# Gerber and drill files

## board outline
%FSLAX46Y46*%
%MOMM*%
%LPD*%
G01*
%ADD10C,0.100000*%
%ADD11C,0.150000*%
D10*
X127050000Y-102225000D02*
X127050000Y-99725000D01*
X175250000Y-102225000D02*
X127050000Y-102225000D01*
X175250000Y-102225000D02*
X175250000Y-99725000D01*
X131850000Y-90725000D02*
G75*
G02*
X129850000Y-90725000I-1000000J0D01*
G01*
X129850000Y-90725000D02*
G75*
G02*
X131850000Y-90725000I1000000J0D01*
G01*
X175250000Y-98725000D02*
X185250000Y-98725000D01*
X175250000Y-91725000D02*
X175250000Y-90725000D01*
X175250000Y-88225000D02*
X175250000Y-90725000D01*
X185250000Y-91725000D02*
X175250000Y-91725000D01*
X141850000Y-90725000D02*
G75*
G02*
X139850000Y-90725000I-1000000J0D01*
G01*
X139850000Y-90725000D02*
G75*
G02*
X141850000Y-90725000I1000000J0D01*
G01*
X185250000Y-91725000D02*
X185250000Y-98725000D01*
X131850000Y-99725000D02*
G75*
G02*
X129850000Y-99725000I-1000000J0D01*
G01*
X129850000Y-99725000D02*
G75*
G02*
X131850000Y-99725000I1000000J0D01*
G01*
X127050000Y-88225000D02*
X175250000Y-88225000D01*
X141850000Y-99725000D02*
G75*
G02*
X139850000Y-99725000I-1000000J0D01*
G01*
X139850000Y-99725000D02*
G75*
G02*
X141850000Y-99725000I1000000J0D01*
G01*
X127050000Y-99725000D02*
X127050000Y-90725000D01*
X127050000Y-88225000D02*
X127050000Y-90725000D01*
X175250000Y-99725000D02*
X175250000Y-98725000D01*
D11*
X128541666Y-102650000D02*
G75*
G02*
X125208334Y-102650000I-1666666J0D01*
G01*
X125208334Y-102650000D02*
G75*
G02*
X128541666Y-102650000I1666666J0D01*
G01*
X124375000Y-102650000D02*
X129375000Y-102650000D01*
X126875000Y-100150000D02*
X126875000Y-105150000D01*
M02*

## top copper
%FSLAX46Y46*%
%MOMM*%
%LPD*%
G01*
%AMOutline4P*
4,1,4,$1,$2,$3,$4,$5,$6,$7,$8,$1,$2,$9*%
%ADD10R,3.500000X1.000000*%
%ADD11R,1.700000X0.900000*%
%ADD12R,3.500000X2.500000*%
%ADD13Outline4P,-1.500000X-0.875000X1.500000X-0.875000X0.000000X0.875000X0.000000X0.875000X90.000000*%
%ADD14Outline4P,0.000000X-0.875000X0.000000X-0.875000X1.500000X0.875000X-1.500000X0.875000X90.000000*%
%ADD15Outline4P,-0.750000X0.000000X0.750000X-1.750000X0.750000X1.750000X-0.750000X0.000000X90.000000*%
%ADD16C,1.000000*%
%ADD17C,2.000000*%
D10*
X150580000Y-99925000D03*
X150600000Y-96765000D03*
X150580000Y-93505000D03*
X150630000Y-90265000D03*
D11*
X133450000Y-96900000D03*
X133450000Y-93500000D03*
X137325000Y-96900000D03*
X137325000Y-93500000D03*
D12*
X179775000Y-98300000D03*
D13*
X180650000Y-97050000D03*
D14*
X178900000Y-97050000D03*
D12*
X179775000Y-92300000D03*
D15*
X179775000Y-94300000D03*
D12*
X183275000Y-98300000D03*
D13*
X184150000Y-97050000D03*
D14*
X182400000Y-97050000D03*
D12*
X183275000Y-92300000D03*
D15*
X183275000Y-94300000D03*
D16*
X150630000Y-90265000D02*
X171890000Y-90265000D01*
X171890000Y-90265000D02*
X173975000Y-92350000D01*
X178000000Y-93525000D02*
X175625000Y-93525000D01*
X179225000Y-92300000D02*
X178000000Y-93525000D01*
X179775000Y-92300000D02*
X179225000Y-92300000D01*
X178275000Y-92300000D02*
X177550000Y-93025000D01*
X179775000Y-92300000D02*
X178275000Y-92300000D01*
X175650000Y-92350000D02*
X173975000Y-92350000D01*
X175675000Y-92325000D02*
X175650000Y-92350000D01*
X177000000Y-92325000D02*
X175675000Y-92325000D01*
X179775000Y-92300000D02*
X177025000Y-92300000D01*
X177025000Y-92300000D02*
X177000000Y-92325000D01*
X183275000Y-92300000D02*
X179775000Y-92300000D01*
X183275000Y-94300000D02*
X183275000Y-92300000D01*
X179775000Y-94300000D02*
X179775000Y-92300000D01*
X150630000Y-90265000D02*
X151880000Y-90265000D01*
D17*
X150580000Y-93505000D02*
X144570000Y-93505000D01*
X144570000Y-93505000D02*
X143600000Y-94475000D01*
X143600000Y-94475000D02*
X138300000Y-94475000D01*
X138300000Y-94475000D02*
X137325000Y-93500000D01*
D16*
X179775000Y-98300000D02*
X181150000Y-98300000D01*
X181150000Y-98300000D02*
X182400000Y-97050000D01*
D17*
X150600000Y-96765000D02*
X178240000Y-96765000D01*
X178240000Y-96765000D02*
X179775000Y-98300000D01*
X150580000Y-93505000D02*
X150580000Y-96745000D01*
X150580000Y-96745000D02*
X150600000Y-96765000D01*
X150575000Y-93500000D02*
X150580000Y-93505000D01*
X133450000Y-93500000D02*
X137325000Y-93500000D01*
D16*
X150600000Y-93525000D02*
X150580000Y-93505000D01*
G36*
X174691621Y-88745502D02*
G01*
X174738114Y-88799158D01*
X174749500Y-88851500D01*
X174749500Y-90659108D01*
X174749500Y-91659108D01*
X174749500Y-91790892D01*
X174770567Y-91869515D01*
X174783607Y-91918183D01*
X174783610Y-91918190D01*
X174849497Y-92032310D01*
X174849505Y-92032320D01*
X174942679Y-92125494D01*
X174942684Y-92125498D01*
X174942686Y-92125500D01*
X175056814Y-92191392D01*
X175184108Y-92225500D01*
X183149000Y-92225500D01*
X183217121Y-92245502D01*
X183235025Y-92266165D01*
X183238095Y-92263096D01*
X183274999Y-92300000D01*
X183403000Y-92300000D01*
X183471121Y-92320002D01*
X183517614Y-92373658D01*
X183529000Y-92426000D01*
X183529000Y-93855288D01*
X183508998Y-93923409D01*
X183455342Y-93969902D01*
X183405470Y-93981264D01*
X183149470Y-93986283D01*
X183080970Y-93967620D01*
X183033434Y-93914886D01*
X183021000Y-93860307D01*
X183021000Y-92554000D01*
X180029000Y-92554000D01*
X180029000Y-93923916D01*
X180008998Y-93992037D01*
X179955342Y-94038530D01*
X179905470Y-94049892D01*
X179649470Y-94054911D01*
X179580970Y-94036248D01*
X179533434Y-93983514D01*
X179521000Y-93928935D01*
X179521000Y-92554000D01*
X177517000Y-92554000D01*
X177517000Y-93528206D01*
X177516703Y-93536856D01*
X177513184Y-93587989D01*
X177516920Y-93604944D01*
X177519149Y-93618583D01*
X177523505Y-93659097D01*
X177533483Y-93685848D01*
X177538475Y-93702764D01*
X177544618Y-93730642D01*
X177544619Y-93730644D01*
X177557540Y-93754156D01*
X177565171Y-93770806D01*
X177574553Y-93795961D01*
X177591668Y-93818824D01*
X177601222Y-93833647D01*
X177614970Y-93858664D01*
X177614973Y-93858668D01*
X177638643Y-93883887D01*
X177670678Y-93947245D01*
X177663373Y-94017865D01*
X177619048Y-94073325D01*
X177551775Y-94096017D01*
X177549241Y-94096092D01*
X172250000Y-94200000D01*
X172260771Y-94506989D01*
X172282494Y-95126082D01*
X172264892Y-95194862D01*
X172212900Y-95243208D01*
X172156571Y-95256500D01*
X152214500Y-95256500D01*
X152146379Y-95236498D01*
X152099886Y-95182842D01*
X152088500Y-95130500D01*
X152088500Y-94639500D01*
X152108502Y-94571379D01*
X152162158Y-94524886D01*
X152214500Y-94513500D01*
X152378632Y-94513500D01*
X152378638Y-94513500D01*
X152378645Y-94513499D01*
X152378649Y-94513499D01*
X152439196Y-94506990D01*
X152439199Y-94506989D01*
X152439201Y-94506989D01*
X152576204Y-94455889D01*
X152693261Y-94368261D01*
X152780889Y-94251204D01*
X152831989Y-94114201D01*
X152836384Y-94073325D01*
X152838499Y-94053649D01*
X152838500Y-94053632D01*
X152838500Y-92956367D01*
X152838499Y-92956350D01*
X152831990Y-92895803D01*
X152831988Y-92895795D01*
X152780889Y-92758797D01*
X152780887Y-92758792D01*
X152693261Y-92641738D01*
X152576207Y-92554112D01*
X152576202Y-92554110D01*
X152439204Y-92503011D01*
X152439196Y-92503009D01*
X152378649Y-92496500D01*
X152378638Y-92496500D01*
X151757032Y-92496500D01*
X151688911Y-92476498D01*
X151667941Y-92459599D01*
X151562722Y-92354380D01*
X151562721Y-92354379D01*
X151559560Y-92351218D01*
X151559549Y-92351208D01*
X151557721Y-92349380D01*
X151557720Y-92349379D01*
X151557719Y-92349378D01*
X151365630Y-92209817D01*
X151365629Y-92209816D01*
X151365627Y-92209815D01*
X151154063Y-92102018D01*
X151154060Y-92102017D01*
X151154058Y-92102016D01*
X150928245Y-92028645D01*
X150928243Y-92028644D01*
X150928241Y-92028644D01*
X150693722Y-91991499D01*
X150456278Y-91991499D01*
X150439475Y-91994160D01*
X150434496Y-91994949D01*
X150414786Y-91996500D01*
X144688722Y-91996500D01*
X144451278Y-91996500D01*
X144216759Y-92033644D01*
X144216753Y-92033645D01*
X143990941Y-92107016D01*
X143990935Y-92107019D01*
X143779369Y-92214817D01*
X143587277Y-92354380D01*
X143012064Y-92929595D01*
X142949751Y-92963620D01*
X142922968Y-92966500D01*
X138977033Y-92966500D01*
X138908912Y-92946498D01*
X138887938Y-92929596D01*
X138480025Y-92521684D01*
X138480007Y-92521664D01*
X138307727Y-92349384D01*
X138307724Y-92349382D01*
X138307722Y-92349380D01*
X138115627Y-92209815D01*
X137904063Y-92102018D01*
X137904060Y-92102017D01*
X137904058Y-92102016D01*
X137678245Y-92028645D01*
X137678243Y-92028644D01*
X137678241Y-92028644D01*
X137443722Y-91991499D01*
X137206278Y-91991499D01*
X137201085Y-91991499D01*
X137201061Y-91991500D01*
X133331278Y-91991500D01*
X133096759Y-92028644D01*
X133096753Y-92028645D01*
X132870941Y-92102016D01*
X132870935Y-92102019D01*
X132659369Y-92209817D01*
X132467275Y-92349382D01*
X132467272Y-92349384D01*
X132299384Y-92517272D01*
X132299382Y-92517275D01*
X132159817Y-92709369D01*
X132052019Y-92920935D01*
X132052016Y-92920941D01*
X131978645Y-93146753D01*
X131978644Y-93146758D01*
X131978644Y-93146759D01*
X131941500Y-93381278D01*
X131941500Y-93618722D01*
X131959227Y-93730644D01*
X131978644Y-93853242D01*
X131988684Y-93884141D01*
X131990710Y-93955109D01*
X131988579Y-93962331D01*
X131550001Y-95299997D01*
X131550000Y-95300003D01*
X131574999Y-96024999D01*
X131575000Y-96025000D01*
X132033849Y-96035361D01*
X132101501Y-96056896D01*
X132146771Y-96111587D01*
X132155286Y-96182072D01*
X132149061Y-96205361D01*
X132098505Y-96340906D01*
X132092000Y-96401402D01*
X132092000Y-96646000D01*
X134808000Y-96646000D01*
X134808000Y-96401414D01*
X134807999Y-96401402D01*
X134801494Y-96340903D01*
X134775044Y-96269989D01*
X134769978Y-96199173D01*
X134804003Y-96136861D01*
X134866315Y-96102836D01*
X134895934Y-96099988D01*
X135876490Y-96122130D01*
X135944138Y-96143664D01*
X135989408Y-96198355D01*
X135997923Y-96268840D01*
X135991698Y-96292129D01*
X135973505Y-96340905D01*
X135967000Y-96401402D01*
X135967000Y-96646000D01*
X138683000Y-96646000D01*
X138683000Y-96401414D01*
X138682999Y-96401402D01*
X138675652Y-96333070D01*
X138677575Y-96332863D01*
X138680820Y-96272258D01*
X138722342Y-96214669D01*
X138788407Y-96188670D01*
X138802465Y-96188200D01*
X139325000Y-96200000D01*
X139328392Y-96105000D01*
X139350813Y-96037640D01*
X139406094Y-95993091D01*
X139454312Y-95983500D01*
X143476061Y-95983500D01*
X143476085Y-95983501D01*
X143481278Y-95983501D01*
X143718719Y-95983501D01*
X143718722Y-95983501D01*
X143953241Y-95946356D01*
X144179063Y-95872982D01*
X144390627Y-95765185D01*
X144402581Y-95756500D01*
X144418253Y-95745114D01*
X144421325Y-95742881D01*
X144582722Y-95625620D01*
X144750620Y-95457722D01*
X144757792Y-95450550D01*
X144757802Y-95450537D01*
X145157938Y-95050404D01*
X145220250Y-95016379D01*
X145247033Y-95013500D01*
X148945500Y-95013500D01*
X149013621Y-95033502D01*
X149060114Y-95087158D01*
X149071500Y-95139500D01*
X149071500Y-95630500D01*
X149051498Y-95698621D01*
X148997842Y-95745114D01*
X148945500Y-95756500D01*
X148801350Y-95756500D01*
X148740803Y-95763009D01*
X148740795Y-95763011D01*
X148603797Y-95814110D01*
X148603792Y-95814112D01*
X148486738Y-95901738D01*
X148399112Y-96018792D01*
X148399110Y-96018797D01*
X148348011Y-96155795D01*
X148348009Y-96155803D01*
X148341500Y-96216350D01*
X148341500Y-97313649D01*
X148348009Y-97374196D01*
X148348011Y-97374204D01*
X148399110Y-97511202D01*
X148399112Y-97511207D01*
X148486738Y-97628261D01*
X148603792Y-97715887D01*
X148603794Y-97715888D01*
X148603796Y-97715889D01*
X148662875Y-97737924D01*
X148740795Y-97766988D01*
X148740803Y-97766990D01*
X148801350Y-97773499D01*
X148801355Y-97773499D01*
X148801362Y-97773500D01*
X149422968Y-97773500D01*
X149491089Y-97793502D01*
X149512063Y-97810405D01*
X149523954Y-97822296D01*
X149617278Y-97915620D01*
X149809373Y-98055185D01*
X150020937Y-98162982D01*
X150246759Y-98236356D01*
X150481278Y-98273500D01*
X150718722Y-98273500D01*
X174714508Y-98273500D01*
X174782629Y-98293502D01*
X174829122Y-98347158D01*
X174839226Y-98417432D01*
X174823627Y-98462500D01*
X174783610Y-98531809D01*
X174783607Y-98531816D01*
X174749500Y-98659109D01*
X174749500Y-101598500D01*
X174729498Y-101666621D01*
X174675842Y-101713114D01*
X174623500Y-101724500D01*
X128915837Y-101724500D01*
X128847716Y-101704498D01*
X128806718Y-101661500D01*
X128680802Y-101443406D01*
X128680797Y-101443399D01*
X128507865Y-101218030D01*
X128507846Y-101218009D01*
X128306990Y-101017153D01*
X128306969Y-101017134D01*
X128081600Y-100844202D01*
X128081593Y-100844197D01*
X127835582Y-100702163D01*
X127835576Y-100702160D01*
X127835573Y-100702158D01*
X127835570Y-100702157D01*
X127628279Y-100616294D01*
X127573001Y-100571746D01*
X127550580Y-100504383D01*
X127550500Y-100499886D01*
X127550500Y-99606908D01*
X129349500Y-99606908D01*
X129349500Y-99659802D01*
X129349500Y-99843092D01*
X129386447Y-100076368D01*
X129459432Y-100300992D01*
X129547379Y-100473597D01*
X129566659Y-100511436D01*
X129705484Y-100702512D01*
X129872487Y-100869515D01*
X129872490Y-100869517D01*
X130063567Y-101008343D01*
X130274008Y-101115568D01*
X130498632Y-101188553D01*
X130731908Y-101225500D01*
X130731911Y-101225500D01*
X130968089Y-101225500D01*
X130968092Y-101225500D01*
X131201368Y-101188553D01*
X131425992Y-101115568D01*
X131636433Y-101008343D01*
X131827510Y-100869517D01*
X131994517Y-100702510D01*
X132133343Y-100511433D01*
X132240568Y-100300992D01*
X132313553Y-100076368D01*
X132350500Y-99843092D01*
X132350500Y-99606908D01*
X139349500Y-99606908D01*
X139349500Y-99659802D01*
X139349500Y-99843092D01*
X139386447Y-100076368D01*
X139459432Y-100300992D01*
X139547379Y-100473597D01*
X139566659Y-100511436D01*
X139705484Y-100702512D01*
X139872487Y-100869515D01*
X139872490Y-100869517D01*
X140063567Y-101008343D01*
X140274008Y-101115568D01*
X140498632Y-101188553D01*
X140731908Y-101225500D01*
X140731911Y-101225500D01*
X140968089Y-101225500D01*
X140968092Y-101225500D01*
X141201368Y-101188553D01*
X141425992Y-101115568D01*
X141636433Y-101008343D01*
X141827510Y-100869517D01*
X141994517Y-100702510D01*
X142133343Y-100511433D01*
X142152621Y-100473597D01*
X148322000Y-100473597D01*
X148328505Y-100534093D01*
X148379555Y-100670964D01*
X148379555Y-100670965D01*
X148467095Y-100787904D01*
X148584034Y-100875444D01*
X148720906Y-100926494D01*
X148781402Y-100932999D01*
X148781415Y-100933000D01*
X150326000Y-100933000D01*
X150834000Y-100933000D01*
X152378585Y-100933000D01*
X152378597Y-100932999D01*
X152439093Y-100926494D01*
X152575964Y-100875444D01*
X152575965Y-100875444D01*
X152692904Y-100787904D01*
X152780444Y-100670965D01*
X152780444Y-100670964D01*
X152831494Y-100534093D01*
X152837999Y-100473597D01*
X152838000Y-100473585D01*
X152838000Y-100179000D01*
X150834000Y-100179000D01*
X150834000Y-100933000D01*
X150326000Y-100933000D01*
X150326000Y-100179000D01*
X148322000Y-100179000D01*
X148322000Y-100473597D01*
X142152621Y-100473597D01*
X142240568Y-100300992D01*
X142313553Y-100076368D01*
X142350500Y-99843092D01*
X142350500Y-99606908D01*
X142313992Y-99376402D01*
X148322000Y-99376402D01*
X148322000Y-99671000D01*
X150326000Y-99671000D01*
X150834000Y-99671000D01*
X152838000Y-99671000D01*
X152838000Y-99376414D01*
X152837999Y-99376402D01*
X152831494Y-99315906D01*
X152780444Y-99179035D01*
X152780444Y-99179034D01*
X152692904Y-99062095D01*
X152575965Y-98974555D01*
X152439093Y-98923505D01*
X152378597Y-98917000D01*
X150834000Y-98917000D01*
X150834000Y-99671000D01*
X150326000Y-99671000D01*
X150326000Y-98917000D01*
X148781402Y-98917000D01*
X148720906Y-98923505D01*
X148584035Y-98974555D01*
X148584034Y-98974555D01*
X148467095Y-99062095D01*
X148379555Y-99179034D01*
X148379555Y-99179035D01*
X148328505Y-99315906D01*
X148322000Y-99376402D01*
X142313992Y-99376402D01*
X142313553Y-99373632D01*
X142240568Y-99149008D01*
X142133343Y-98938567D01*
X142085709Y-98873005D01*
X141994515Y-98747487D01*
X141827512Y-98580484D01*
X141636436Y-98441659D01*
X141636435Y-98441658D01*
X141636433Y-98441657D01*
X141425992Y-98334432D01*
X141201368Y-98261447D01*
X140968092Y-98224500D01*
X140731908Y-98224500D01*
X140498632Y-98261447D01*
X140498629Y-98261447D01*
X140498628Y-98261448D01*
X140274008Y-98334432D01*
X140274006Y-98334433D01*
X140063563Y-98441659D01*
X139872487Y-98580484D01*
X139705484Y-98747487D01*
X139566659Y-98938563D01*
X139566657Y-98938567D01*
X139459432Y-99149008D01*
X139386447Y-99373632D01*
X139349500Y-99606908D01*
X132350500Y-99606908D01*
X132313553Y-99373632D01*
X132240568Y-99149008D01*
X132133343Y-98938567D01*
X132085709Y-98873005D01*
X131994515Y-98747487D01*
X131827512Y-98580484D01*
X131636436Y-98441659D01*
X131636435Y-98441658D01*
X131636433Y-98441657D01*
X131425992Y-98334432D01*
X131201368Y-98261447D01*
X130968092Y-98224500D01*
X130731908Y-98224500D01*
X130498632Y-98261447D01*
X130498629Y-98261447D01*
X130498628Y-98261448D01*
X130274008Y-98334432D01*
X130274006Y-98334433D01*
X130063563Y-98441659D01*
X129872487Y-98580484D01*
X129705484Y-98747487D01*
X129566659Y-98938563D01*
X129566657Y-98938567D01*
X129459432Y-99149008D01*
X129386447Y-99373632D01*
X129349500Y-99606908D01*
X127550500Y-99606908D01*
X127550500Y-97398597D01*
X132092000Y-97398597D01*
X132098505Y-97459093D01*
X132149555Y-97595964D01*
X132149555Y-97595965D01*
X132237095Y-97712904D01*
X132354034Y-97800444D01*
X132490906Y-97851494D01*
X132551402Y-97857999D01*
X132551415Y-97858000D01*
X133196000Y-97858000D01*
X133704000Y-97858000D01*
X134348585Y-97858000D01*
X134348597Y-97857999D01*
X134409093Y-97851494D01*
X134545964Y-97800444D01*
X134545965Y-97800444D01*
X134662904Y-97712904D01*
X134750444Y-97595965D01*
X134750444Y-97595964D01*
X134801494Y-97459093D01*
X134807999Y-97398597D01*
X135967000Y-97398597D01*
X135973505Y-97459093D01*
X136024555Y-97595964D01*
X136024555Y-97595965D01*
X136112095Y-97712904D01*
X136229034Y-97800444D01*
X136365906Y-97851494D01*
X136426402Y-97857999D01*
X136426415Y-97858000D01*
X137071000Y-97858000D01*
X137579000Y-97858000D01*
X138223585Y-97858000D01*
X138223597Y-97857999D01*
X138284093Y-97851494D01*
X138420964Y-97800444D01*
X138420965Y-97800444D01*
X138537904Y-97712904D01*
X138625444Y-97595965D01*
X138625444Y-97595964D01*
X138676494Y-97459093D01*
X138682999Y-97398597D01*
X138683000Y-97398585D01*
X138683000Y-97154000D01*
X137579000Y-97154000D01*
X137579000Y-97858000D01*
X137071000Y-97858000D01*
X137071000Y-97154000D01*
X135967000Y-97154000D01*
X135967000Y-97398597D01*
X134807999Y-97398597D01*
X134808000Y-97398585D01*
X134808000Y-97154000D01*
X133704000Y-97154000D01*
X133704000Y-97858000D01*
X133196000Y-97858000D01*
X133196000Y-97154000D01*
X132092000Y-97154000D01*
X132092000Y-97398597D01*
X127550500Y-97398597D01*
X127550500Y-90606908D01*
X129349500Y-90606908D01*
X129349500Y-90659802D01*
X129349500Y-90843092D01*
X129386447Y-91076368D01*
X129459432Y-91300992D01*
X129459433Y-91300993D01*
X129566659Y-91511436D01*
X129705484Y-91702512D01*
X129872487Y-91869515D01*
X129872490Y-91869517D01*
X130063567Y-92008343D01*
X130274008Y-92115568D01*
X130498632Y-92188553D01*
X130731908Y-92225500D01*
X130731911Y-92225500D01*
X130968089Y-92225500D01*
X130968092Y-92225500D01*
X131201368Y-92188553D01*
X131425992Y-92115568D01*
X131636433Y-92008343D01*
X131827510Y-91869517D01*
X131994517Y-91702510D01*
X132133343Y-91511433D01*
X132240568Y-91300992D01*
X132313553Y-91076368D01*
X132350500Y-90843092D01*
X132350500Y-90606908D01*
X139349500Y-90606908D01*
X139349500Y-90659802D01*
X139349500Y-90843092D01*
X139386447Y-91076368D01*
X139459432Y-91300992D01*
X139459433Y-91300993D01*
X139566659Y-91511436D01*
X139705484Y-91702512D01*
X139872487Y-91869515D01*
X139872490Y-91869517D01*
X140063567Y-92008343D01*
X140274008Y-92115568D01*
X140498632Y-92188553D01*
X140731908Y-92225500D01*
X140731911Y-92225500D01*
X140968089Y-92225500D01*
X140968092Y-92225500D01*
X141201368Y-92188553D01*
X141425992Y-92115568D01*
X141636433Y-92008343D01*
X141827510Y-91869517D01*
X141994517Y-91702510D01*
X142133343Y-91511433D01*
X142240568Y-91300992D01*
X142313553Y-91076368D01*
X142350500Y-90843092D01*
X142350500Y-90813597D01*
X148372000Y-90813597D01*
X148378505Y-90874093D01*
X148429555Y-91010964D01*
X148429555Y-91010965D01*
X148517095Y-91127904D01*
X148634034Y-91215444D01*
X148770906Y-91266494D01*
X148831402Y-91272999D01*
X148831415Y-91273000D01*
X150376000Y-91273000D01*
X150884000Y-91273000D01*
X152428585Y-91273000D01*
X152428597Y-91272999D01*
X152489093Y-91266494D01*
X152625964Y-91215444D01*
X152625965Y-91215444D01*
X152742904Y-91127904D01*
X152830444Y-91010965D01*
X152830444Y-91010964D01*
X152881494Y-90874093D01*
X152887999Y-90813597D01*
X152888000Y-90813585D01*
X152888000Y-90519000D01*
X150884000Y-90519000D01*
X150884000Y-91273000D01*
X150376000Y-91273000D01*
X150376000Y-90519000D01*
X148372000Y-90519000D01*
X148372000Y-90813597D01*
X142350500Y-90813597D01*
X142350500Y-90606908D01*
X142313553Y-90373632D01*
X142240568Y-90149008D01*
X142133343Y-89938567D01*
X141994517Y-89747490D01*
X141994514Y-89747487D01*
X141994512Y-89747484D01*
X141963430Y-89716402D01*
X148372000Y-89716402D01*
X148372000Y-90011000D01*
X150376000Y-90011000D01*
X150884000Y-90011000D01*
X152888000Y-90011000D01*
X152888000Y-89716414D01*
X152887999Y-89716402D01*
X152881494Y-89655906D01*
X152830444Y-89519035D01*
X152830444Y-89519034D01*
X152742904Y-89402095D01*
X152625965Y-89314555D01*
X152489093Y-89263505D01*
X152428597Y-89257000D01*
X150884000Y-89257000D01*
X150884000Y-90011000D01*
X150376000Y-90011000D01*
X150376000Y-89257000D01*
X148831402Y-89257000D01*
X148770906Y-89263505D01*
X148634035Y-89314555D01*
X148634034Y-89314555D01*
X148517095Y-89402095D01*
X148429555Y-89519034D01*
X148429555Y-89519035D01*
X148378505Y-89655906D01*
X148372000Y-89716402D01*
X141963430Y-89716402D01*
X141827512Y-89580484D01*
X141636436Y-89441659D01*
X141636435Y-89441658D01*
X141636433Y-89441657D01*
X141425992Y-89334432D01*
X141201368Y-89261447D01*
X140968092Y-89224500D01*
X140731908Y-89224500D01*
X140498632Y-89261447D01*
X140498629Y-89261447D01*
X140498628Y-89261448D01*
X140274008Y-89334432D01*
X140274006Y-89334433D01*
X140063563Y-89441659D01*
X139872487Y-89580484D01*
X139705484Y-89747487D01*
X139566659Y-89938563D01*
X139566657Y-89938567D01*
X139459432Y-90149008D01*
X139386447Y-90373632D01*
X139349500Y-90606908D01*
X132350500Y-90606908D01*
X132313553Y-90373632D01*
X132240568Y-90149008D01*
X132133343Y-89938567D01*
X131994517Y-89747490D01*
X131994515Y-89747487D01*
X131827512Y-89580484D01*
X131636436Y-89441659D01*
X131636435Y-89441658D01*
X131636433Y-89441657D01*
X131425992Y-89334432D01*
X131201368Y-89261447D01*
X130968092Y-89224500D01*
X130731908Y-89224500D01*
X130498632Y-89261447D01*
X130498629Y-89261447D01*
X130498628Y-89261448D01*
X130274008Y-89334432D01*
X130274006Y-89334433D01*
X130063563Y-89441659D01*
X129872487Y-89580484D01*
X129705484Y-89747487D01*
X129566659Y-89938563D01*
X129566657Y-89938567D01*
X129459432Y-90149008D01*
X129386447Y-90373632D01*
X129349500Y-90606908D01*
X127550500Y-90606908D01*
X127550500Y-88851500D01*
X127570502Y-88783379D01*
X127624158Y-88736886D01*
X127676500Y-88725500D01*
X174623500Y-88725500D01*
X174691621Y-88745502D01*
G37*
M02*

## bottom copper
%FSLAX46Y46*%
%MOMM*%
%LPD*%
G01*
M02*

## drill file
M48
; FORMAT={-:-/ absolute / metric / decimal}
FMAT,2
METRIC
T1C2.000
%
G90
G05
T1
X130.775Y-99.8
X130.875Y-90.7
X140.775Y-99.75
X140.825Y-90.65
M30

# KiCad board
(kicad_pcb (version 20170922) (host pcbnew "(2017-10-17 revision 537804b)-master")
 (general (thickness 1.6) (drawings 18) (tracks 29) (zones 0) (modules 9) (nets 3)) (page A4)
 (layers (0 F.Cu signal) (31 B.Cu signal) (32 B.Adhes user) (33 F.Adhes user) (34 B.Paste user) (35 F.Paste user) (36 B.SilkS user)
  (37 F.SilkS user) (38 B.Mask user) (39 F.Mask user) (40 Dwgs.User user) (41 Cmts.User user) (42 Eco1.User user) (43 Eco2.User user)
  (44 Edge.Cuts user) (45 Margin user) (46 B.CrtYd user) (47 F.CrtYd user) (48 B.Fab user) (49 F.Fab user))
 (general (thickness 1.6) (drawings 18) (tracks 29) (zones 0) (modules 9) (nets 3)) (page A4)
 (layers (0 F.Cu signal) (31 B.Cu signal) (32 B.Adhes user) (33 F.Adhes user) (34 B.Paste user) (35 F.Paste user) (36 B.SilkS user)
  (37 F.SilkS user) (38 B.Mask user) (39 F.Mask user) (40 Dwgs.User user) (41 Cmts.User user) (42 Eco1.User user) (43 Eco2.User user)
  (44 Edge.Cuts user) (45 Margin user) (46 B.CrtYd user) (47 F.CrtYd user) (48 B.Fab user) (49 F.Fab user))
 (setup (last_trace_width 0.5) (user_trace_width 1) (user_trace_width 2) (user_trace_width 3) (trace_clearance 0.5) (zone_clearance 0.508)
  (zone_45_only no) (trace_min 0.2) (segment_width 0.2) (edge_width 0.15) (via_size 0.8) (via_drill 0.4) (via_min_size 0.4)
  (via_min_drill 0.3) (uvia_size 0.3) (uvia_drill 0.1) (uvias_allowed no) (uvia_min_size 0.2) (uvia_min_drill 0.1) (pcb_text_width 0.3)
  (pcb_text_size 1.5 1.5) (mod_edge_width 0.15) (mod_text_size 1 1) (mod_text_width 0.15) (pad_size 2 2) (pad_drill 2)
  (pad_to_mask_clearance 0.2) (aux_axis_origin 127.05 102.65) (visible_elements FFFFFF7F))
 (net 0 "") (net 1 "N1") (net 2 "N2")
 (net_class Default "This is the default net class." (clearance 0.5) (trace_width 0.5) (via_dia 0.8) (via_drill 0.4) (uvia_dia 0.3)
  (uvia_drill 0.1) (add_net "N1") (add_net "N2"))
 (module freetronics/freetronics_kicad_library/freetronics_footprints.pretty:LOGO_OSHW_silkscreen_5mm (layer F.Cu) (at 166.775 94.425)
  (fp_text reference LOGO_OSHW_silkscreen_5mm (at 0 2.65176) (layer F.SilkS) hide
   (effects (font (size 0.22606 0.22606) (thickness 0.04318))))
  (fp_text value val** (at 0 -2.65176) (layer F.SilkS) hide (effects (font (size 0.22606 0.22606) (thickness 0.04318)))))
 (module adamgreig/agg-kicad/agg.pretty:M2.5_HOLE (layer F.Cu) (at 140.775 99.75)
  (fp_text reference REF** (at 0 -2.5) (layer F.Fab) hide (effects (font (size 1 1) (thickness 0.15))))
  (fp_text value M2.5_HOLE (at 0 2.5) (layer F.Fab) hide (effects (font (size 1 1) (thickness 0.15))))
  (pad "" np_thru_hole circle (at 0 0) (size 2 2) (drill 2) (layers *.Cu F.Mask)))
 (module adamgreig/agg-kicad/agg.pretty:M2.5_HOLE (layer F.Cu) (at 130.775 99.8)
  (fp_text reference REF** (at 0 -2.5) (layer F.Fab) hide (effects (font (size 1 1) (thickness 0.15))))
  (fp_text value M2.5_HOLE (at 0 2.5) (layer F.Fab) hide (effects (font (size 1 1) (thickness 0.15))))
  (pad "" np_thru_hole circle (at 0 0) (size 2 2) (drill 2) (layers *.Cu F.Mask)))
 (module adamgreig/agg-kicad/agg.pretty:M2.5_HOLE (layer F.Cu) (at 140.825 90.65)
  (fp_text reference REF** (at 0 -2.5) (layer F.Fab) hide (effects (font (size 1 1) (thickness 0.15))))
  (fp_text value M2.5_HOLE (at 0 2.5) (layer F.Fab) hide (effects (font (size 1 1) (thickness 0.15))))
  (pad "" np_thru_hole circle (at 0 0) (size 2 2) (drill 2) (layers *.Cu F.Mask)))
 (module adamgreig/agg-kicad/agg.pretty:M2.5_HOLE (layer F.Cu) (at 130.875 90.7)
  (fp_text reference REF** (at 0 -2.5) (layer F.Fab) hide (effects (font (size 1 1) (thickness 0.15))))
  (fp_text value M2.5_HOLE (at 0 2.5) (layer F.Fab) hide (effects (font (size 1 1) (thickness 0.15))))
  (pad "" np_thru_hole circle (at 0 0) (size 2 2) (drill 2) (layers *.Cu F.Mask)))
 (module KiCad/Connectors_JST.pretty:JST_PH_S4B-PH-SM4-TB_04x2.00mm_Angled (layer F.Cu) (at 153.5 95.025 90)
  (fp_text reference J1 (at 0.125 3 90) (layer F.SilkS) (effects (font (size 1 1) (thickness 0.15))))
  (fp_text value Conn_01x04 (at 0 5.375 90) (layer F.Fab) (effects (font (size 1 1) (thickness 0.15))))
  (pad 1 smd rect (at -4.9 -2.92 90) (size 1 3.5) (layers F.Cu F.Paste F.Mask) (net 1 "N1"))
  (pad 2 smd rect (at -1.74 -2.9 90) (size 1 3.5) (layers F.Cu F.Paste F.Mask) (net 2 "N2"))
  (pad 3 smd rect (at 1.52 -2.92 90) (size 1 3.5) (layers F.Cu F.Paste F.Mask) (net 2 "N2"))
  (pad 4 smd rect (at 4.76 -2.87 90) (size 1 3.5) (layers F.Cu F.Paste F.Mask) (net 1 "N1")))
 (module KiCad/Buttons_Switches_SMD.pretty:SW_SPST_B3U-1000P (layer F.Cu) (at 133.45 95.2 90)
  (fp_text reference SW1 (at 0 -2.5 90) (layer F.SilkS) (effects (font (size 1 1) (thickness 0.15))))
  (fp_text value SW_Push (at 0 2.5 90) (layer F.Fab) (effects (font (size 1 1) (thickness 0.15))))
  (pad 1 smd rect (at -1.7 0 90) (size 0.9 1.7) (layers F.Cu F.Paste F.Mask) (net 1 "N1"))
  (pad 2 smd rect (at 1.7 0 90) (size 0.9 1.7) (layers F.Cu F.Paste F.Mask) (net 2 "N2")))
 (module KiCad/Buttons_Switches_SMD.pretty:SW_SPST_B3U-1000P (layer F.Cu) (at 137.325 95.2 270)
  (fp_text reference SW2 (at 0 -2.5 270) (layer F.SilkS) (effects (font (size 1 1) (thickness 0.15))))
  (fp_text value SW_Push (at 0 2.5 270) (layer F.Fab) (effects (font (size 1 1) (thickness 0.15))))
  (pad 2 smd rect (at 1.7 0 270) (size 0.9 1.7) (layers F.Cu F.Paste F.Mask) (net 1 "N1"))
  (pad 1 smd rect (at -1.7 0 270) (size 0.9 1.7) (layers F.Cu F.Paste F.Mask) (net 2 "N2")))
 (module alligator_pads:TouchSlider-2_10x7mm (layer F.Cu) (at 181.525 95.3 90)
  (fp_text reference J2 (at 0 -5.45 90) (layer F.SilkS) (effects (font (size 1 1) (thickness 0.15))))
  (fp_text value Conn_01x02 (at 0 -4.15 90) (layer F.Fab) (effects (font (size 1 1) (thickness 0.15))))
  (pad 1 smd rect (at -3 -1.75 90) (size 2.5 3.5) (layers F.Cu F.Mask) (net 2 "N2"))
  (pad 1 smd trapezoid (at -1.75 -0.875 90) (size 1.5 1.75) (rect_delta 0 1.5) (layers F.Cu F.Mask) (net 2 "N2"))
  (pad 1 smd trapezoid (at -1.75 -2.625 90) (size 1.5 1.75) (rect_delta 0 -1.5) (layers F.Cu F.Mask) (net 2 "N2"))
  (pad 2 smd rect (at 3 -1.75 90) (size 2.5 3.5) (layers F.Cu F.Mask) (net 1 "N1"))
  (pad 2 smd trapezoid (at 1 -1.75 90) (size 1.5 1.75) (rect_delta -1.75 0) (layers F.Cu F.Mask) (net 1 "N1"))
  (pad 1 smd rect (at -3 1.75 90) (size 2.5 3.5) (layers F.Cu F.Mask) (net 2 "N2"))
  (pad 1 smd trapezoid (at -1.75 2.625 90) (size 1.5 1.75) (rect_delta 0 1.5) (layers F.Cu F.Mask) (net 2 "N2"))
  (pad 1 smd trapezoid (at -1.75 0.875 90) (size 1.5 1.75) (rect_delta 0 -1.5) (layers F.Cu F.Mask) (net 2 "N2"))
  (pad 2 smd rect (at 3 1.75 90) (size 2.5 3.5) (layers F.Cu F.Mask) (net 1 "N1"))
  (pad 2 smd trapezoid (at 1 1.75 90) (size 1.5 1.75) (rect_delta -1.75 0) (layers F.Cu F.Mask) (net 1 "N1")))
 (gr_line (start 127.05 102.225) (end 127.05 99.725) (layer Edge.Cuts) (width 0.1))
 (gr_line (start 175.25 102.225) (end 127.05 102.225) (layer Edge.Cuts) (width 0.1))
 (gr_line (start 175.25 102.225) (end 175.25 99.725) (layer Edge.Cuts) (width 0.1))
 (gr_circle (center 130.85 90.725) (end 131.85 90.725) (layer Edge.Cuts) (width 0.1))
 (gr_line (start 175.25 98.725) (end 185.25 98.725) (layer Edge.Cuts) (width 0.1))
 (gr_line (start 175.25 91.725) (end 175.25 90.725) (layer Edge.Cuts) (width 0.1))
 (gr_line (start 175.25 88.225) (end 175.25 90.725) (layer Edge.Cuts) (width 0.1))
 (gr_line (start 185.25 91.725) (end 175.25 91.725) (layer Edge.Cuts) (width 0.1))
 (gr_circle (center 140.85 90.725) (end 141.85 90.725) (layer Edge.Cuts) (width 0.1))
 (gr_line (start 185.25 91.725) (end 185.25 98.725) (layer Edge.Cuts) (width 0.1))
 (gr_circle (center 130.85 99.725) (end 131.85 99.725) (layer Edge.Cuts) (width 0.1))
 (gr_line (start 127.05 88.225) (end 175.25 88.225) (layer Edge.Cuts) (width 0.1))
 (gr_circle (center 140.85 99.725) (end 141.85 99.725) (layer Edge.Cuts) (width 0.1))
 (gr_line (start 127.05 99.725) (end 127.05 90.725) (layer Edge.Cuts) (width 0.1))
 (gr_line (start 127.05 88.225) (end 127.05 90.725) (layer Edge.Cuts) (width 0.1))
 (gr_line (start 175.25 99.725) (end 175.25 98.725) (layer Edge.Cuts) (width 0.1))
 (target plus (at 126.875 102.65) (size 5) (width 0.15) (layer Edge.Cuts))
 (segment (start 150.63 90.265) (end 171.89 90.265) (width 1) (layer F.Cu) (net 1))
 (segment (start 171.89 90.265) (end 173.975 92.35) (width 1) (layer F.Cu) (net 1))
 (segment (start 178 93.525) (end 175.625 93.525) (width 1) (layer F.Cu) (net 1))
 (segment (start 179.225 92.3) (end 178 93.525) (width 1) (layer F.Cu) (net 1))
 (segment (start 179.775 92.3) (end 179.225 92.3) (width 1) (layer F.Cu) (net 1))
 (segment (start 178.275 92.3) (end 177.55 93.025) (width 1) (layer F.Cu) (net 1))
 (segment (start 179.775 92.3) (end 178.275 92.3) (width 1) (layer F.Cu) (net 1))
 (segment (start 175.65 92.35) (end 173.975 92.35) (width 1) (layer F.Cu) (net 1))
 (segment (start 175.675 92.325) (end 175.65 92.35) (width 1) (layer F.Cu) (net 1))
 (segment (start 177 92.325) (end 175.675 92.325) (width 1) (layer F.Cu) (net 1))
 (segment (start 179.775 92.3) (end 177.025 92.3) (width 1) (layer F.Cu) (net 1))
 (segment (start 177.025 92.3) (end 177 92.325) (width 1) (layer F.Cu) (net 1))
 (segment (start 183.275 92.3) (end 179.775 92.3) (width 1) (layer F.Cu) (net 1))
 (segment (start 183.275 94.3) (end 183.275 92.3) (width 1) (layer F.Cu) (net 1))
 (segment (start 179.775 94.3) (end 179.775 92.3) (width 1) (layer F.Cu) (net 1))
 (segment (start 150.63 90.265) (end 151.88 90.265) (width 1) (layer F.Cu) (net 1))
 (segment (start 150.58 93.505) (end 144.57 93.505) (width 2) (layer F.Cu) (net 2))
 (segment (start 144.57 93.505) (end 143.6 94.475) (width 2) (layer F.Cu) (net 2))
 (segment (start 143.6 94.475) (end 138.3 94.475) (width 2) (layer F.Cu) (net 2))
 (segment (start 138.3 94.475) (end 137.325 93.5) (width 2) (layer F.Cu) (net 2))
 (segment (start 179.775 98.3) (end 181.15 98.3) (width 1) (layer F.Cu) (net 2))
 (segment (start 181.15 98.3) (end 182.4 97.05) (width 1) (layer F.Cu) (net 2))
 (segment (start 150.6 96.765) (end 178.24 96.765) (width 2) (layer F.Cu) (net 2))
 (segment (start 178.24 96.765) (end 179.775 98.3) (width 2) (layer F.Cu) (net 2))
 (segment (start 150.58 93.505) (end 150.58 96.745) (width 2) (layer F.Cu) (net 2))
 (segment (start 150.58 96.745) (end 150.6 96.765) (width 2) (layer F.Cu) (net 2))
 (segment (start 150.575 93.5) (end 150.58 93.505) (width 2) (layer F.Cu) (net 2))
 (segment (start 133.45 93.5) (end 137.325 93.5) (width 2) (layer F.Cu) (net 2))
 (segment (start 150.6 93.525) (end 150.58 93.505) (width 1) (layer F.Cu) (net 2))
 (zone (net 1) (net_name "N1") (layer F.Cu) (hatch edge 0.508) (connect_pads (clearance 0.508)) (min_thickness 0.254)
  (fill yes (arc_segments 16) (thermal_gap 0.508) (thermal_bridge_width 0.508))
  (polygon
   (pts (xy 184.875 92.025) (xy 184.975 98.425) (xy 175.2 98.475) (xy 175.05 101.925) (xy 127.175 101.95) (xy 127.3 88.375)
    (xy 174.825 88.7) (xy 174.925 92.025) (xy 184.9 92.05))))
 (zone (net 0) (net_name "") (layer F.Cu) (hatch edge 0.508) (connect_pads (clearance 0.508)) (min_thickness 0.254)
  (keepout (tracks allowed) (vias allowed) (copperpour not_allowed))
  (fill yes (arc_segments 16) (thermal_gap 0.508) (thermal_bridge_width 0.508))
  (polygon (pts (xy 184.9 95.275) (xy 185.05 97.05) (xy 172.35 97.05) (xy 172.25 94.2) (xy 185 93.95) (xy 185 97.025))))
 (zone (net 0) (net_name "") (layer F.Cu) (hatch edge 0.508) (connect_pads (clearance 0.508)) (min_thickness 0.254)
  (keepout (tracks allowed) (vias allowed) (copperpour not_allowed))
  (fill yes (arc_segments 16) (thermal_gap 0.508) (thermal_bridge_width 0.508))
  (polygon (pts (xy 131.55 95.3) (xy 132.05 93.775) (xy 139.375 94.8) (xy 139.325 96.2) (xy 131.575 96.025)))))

